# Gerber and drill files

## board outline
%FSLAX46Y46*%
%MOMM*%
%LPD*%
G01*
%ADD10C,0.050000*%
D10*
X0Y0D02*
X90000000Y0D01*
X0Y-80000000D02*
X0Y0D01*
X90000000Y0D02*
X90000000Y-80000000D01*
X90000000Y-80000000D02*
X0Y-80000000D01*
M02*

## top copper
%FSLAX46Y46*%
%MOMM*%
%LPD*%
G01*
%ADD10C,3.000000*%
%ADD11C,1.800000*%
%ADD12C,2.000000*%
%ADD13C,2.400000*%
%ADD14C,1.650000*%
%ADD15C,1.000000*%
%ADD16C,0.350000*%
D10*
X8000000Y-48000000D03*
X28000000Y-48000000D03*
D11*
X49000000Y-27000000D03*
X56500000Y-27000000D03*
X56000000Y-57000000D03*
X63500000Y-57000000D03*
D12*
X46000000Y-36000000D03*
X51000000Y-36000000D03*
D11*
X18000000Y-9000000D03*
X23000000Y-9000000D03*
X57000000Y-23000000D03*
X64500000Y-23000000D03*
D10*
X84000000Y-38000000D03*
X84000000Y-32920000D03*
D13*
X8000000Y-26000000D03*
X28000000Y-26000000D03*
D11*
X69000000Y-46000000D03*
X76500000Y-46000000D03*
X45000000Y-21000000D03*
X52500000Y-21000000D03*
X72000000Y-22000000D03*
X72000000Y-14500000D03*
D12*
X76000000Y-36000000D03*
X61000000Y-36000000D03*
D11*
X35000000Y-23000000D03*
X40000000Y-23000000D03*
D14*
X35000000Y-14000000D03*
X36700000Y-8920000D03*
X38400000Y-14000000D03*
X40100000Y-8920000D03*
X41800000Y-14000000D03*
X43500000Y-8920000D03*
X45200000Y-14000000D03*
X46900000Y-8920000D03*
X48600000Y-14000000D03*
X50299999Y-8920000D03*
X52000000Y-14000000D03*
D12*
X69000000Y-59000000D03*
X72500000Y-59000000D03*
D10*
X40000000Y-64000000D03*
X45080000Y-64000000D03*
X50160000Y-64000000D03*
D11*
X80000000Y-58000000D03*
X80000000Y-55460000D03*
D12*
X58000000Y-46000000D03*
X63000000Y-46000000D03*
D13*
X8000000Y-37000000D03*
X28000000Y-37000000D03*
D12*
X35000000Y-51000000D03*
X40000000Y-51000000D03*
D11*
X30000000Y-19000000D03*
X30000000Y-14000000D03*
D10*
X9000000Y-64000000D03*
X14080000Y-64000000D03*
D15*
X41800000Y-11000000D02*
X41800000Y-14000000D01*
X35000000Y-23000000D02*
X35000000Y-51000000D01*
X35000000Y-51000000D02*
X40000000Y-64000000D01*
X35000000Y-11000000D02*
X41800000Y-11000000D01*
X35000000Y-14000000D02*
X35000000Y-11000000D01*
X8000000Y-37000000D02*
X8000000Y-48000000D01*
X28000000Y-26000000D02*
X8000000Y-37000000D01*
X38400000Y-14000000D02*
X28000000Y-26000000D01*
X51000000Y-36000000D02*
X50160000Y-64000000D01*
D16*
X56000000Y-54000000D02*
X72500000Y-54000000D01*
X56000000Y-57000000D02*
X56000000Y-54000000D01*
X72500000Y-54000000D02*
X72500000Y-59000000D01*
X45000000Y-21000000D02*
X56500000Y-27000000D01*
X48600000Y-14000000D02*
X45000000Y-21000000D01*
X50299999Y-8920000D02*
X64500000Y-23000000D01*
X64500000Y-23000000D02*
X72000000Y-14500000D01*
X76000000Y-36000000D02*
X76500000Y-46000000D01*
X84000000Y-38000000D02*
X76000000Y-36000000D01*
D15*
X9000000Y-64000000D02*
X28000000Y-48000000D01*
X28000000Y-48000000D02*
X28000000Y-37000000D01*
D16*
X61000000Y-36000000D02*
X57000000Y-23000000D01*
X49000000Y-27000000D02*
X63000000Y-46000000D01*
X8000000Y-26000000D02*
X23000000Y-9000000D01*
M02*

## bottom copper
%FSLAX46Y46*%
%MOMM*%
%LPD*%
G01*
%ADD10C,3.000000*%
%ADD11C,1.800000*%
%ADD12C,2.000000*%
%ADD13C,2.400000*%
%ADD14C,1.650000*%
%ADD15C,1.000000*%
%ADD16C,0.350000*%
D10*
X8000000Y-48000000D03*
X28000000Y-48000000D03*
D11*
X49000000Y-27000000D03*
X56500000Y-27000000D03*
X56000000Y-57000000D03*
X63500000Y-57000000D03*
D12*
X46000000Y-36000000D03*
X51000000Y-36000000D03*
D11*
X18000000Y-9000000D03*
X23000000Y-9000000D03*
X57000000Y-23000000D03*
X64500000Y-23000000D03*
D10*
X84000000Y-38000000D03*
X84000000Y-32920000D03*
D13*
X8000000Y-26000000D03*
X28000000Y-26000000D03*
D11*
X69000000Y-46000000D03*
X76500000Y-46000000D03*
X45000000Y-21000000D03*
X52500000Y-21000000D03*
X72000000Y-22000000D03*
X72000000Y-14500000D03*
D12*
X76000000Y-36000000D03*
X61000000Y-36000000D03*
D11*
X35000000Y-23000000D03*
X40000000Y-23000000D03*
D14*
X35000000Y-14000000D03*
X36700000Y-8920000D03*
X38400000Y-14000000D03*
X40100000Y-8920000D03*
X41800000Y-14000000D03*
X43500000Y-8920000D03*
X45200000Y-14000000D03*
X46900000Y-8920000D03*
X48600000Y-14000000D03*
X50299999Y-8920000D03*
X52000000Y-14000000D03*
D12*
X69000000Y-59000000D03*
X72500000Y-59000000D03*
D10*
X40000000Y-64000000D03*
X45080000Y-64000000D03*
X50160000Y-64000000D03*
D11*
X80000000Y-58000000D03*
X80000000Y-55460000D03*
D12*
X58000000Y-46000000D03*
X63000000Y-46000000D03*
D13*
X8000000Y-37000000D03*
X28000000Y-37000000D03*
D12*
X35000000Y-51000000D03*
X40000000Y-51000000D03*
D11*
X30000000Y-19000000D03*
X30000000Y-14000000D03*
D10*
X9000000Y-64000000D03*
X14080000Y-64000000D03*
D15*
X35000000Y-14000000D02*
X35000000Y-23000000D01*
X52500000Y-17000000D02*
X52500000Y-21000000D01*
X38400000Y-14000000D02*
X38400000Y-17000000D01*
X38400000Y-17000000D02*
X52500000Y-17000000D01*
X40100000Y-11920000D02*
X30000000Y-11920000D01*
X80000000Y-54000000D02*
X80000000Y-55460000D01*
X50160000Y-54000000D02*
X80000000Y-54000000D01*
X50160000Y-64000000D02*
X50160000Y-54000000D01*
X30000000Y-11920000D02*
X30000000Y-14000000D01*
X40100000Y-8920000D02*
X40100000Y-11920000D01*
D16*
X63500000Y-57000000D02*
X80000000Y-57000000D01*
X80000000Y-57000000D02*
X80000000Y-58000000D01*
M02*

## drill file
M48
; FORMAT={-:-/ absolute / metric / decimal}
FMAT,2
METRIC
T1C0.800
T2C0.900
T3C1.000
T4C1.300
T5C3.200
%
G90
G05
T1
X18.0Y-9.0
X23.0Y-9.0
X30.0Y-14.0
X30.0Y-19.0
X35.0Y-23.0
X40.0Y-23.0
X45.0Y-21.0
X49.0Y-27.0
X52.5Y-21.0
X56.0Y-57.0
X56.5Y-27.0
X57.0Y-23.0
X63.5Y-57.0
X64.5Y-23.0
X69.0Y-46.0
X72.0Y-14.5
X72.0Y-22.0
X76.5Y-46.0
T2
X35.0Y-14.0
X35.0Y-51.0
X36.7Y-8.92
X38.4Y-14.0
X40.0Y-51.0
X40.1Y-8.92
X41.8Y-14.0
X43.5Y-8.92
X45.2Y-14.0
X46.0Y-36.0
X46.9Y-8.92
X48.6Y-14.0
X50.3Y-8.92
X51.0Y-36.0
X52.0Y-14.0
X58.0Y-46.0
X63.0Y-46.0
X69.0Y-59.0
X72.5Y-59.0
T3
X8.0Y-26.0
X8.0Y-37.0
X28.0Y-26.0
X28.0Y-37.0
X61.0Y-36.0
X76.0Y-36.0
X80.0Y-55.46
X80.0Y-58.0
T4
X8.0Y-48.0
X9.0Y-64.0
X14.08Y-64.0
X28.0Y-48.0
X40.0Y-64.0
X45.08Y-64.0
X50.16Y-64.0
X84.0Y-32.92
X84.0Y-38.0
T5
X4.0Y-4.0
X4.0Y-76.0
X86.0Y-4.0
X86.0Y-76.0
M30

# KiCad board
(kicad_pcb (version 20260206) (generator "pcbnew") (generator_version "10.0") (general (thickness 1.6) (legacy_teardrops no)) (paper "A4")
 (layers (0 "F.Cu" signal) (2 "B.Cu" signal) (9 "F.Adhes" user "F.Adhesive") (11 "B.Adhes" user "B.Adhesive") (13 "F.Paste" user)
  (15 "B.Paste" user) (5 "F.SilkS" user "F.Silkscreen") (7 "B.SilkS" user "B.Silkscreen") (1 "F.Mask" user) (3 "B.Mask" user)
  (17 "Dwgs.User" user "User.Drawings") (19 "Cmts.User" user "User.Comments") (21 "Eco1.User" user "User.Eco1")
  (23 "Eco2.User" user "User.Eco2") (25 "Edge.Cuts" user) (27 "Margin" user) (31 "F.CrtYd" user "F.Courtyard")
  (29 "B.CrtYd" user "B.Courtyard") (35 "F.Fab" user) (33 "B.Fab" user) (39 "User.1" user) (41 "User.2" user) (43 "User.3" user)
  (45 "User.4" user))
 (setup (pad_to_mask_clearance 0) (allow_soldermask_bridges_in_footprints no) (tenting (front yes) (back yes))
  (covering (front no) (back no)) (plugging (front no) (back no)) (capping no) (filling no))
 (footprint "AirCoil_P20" (layer "F.Cu") (at 8 48)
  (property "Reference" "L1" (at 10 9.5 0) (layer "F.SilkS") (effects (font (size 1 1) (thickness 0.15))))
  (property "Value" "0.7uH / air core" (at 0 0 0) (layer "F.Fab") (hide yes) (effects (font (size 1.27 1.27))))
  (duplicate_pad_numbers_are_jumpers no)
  (pad "1" thru_hole circle (at 0 0) (size 3 3) (drill 1.3) (layers "*.Cu" "*.Mask") (remove_unused_layers no) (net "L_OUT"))
  (pad "2" thru_hole circle (at 20 0) (size 3 3) (drill 1.3) (layers "*.Cu" "*.Mask") (remove_unused_layers no) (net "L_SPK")))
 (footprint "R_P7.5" (layer "F.Cu") (at 49 27)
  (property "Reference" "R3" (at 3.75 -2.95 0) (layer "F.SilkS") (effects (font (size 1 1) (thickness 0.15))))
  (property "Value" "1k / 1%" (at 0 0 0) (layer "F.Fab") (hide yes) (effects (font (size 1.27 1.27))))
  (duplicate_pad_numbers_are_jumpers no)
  (pad "1" thru_hole circle (at 0 0) (size 1.8 1.8) (drill 0.8) (layers "*.Cu" "*.Mask") (remove_unused_layers no) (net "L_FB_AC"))
  (pad "2" thru_hole circle (at 7.5 0) (size 1.8 1.8) (drill 0.8) (layers "*.Cu" "*.Mask") (remove_unused_layers no) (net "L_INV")))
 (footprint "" (layer "F.Cu") (at 4 4)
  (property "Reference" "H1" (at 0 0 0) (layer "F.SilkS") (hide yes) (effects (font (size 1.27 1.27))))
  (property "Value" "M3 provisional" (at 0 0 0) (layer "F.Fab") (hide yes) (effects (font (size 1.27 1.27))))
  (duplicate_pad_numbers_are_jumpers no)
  (pad "" np_thru_hole circle (at 0 0) (size 3.2 3.2) (drill 3.2) (layers "*.Cu" "*.Mask")))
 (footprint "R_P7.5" (layer "F.Cu") (at 56 57)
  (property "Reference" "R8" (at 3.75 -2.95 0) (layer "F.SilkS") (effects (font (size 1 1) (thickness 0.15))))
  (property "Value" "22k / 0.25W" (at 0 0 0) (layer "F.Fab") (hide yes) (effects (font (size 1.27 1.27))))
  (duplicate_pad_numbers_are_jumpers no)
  (pad "1" thru_hole circle (at 0 0) (size 1.8 1.8) (drill 0.8) (layers "*.Cu" "*.Mask") (remove_unused_layers no) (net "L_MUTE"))
  (pad "2" thru_hole circle (at 7.5 0) (size 1.8 1.8) (drill 0.8) (layers "*.Cu" "*.Mask") (remove_unused_layers no) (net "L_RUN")))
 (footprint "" (layer "F.Cu") (at 86 4)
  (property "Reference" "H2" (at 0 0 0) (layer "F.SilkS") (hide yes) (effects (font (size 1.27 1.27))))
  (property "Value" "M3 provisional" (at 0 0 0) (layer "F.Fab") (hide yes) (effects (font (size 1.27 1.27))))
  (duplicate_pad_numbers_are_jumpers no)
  (pad "" np_thru_hole circle (at 0 0) (size 3.2 3.2) (drill 3.2) (layers "*.Cu" "*.Mask")))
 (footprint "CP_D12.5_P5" (layer "F.Cu") (at 46 36)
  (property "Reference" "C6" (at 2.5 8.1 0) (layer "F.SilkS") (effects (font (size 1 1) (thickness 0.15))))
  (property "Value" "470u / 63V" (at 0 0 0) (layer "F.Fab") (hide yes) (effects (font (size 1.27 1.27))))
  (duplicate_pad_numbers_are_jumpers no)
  (pad "1" thru_hole circle (at 0 0) (size 2 2) (drill 0.9) (layers "*.Cu" "*.Mask") (remove_unused_layers no) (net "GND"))
  (pad "2" thru_hole circle (at 5 0) (size 2 2) (drill 0.9) (layers "*.Cu" "*.Mask") (remove_unused_layers no) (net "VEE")))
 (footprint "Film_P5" (layer "F.Cu") (at 18 9)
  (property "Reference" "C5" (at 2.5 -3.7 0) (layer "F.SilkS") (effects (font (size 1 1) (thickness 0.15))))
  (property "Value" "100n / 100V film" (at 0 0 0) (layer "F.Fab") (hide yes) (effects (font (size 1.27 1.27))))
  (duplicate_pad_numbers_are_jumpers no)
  (pad "1" thru_hole circle (at 0 0) (size 1.8 1.8) (drill 0.8) (layers "*.Cu" "*.Mask") (remove_unused_layers no) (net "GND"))
  (pad "2" thru_hole circle (at 5 0) (size 1.8 1.8) (drill 0.8) (layers "*.Cu" "*.Mask") (remove_unused_layers no) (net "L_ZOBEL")))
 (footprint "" (layer "F.Cu") (at 4 76)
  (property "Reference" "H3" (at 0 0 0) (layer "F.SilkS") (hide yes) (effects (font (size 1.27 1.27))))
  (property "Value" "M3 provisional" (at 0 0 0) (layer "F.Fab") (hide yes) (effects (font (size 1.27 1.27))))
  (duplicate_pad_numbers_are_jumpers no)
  (pad "" np_thru_hole circle (at 0 0) (size 3.2 3.2) (drill 3.2) (layers "*.Cu" "*.Mask")))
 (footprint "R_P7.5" (layer "F.Cu") (at 57 23)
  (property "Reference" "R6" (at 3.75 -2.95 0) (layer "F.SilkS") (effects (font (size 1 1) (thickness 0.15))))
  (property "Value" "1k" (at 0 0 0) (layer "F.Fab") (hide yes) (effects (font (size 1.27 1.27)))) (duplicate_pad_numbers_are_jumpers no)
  (pad "1" thru_hole circle (at 0 0) (size 1.8 1.8) (drill 0.8) (layers "*.Cu" "*.Mask") (remove_unused_layers no) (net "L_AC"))
  (pad "2" thru_hole circle (at 7.5 0) (size 1.8 1.8) (drill 0.8) (layers "*.Cu" "*.Mask") (remove_unused_layers no) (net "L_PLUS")))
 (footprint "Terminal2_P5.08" (layer "F.Cu") (at 84 38 90)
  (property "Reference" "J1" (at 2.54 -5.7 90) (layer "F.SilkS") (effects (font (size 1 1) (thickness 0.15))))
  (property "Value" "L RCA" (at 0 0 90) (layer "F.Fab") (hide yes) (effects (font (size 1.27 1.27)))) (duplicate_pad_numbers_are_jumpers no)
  (pad "1" thru_hole circle (at 0 0 90) (size 3 3) (drill 1.3) (layers "*.Cu" "*.Mask") (remove_unused_layers no) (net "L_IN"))
  (pad "2" thru_hole circle (at 5.08 0 90) (size 3 3) (drill 1.3) (layers "*.Cu" "*.Mask") (remove_unused_layers no) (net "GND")))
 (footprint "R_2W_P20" (layer "F.Cu") (at 8 26)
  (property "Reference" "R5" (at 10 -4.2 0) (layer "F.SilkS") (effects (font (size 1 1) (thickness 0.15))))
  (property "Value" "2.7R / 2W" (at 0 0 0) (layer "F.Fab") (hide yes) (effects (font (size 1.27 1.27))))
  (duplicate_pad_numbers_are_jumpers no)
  (pad "1" thru_hole circle (at 0 0) (size 2.4 2.4) (drill 1) (layers "*.Cu" "*.Mask") (remove_unused_layers no) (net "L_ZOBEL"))
  (pad "2" thru_hole circle (at 20 0) (size 2.4 2.4) (drill 1) (layers "*.Cu" "*.Mask") (remove_unused_layers no) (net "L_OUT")))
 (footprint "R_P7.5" (layer "F.Cu") (at 69 46)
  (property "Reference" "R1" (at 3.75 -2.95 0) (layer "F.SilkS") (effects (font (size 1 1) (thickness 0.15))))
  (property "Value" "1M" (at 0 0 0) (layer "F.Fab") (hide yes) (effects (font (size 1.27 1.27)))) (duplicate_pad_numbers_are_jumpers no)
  (pad "1" thru_hole circle (at 0 0) (size 1.8 1.8) (drill 0.8) (layers "*.Cu" "*.Mask") (remove_unused_layers no) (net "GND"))
  (pad "2" thru_hole circle (at 7.5 0) (size 1.8 1.8) (drill 0.8) (layers "*.Cu" "*.Mask") (remove_unused_layers no) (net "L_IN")))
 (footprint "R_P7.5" (layer "F.Cu") (at 45 21)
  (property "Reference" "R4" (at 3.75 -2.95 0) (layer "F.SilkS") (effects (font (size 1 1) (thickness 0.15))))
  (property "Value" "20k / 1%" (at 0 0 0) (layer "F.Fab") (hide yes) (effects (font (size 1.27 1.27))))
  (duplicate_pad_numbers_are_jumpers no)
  (pad "1" thru_hole circle (at 0 0) (size 1.8 1.8) (drill 0.8) (layers "*.Cu" "*.Mask") (remove_unused_layers no) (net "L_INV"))
  (pad "2" thru_hole circle (at 7.5 0) (size 1.8 1.8) (drill 0.8) (layers "*.Cu" "*.Mask") (remove_unused_layers no) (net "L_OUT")))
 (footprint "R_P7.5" (layer "F.Cu") (at 72 22 90)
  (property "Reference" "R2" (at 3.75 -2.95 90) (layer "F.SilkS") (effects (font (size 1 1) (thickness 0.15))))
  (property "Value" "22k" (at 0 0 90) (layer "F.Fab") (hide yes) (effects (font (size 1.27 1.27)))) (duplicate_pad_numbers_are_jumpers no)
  (pad "1" thru_hole circle (at 0 0 90) (size 1.8 1.8) (drill 0.8) (layers "*.Cu" "*.Mask") (remove_unused_layers no) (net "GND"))
  (pad "2" thru_hole circle (at 7.5 0 90) (size 1.8 1.8) (drill 0.8) (layers "*.Cu" "*.Mask") (remove_unused_layers no) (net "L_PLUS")))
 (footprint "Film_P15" (layer "F.Cu") (at 76 36 180)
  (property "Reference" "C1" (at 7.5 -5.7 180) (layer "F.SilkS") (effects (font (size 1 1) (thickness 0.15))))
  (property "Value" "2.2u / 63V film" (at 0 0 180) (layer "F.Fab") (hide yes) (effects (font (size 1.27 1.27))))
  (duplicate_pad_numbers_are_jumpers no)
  (pad "1" thru_hole circle (at 0 0 180) (size 2 2) (drill 1) (layers "*.Cu" "*.Mask") (remove_unused_layers no) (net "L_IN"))
  (pad "2" thru_hole circle (at 15 0 180) (size 2 2) (drill 1) (layers "*.Cu" "*.Mask") (remove_unused_layers no) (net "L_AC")))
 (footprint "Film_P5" (layer "F.Cu") (at 35 23)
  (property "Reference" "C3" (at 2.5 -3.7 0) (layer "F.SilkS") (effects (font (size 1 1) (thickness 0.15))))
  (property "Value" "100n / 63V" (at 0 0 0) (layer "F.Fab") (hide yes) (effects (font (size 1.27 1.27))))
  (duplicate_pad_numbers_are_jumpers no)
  (pad "1" thru_hole circle (at 0 0) (size 1.8 1.8) (drill 0.8) (layers "*.Cu" "*.Mask") (remove_unused_layers no) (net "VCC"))
  (pad "2" thru_hole circle (at 5 0) (size 1.8 1.8) (drill 0.8) (layers "*.Cu" "*.Mask") (remove_unused_layers no) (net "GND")))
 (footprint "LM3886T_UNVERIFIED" (layer "F.Cu") (at 35 14)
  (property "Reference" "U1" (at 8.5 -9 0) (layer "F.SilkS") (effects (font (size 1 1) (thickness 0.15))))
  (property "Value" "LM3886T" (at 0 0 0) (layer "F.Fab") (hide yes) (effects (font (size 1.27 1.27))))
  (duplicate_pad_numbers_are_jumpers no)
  (pad "1" thru_hole circle (at 0 0) (size 1.65 1.65) (drill 0.9) (layers "*.Cu" "*.Mask") (remove_unused_layers no) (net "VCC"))
  (pad "2" thru_hole circle (at 1.7 -5.08) (size 1.65 1.65) (drill 0.9) (layers "*.Cu" "*.Mask") (remove_unused_layers no)
   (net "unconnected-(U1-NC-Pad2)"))
  (pad "3" thru_hole circle (at 3.4 0) (size 1.65 1.65) (drill 0.9) (layers "*.Cu" "*.Mask") (remove_unused_layers no) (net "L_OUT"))
  (pad "4" thru_hole circle (at 5.1 -5.08) (size 1.65 1.65) (drill 0.9) (layers "*.Cu" "*.Mask") (remove_unused_layers no) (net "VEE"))
  (pad "5" thru_hole circle (at 6.8 0) (size 1.65 1.65) (drill 0.9) (layers "*.Cu" "*.Mask") (remove_unused_layers no) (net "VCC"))
  (pad "6" thru_hole circle (at 8.5 -5.08) (size 1.65 1.65) (drill 0.9) (layers "*.Cu" "*.Mask") (remove_unused_layers no)
   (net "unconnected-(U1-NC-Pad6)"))
  (pad "7" thru_hole circle (at 10.2 0) (size 1.65 1.65) (drill 0.9) (layers "*.Cu" "*.Mask") (remove_unused_layers no) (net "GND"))
  (pad "8" thru_hole circle (at 11.9 -5.08) (size 1.65 1.65) (drill 0.9) (layers "*.Cu" "*.Mask") (remove_unused_layers no) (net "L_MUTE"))
  (pad "9" thru_hole circle (at 13.6 0) (size 1.65 1.65) (drill 0.9) (layers "*.Cu" "*.Mask") (remove_unused_layers no) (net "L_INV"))
  (pad "10" thru_hole circle (at 15.299999 -5.08) (size 1.65 1.65) (drill 0.9) (layers "*.Cu" "*.Mask") (remove_unused_layers no)
   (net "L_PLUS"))
  (pad "11" thru_hole circle (at 17 0) (size 1.65 1.65) (drill 0.9) (layers "*.Cu" "*.Mask") (remove_unused_layers no)
   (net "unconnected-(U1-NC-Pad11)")))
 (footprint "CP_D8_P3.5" (layer "F.Cu") (at 69 59)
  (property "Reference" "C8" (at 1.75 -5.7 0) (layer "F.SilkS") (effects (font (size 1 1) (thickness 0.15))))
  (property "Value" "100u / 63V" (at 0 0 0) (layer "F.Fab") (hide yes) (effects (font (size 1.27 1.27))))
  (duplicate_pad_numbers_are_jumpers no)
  (pad "1" thru_hole circle (at 0 0) (size 2 2) (drill 0.9) (layers "*.Cu" "*.Mask") (remove_unused_layers no) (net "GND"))
  (pad "2" thru_hole circle (at 3.5 0) (size 2 2) (drill 0.9) (layers "*.Cu" "*.Mask") (remove_unused_layers no) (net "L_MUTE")))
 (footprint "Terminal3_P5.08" (layer "F.Cu") (at 40 64)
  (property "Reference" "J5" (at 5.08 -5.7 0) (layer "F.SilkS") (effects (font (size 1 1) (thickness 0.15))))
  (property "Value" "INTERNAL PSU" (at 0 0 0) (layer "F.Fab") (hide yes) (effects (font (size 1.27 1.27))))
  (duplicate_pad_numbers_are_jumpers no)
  (pad "1" thru_hole circle (at 0 0) (size 3 3) (drill 1.3) (layers "*.Cu" "*.Mask") (remove_unused_layers no) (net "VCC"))
  (pad "2" thru_hole circle (at 5.08 0) (size 3 3) (drill 1.3) (layers "*.Cu" "*.Mask") (remove_unused_layers no) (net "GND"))
  (pad "3" thru_hole circle (at 10.16 0) (size 3 3) (drill 1.3) (layers "*.Cu" "*.Mask") (remove_unused_layers no) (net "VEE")))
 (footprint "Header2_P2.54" (layer "F.Cu") (at 80 58 90)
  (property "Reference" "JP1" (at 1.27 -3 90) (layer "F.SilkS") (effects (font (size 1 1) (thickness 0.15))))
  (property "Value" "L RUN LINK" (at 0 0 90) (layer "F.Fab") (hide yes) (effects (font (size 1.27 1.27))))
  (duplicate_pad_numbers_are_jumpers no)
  (pad "1" thru_hole circle (at 0 0 90) (size 1.8 1.8) (drill 1) (layers "*.Cu" "*.Mask") (remove_unused_layers no) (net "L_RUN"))
  (pad "2" thru_hole circle (at 2.54 0 90) (size 1.8 1.8) (drill 1) (layers "*.Cu" "*.Mask") (remove_unused_layers no) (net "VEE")))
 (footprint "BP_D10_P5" (layer "F.Cu") (at 58 46)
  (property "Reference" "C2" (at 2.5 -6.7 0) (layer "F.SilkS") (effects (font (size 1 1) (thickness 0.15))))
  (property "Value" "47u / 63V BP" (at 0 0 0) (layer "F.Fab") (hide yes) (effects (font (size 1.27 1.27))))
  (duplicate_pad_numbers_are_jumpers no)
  (pad "1" thru_hole circle (at 0 0) (size 2 2) (drill 0.9) (layers "*.Cu" "*.Mask") (remove_unused_layers no) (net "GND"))
  (pad "2" thru_hole circle (at 5 0) (size 2 2) (drill 0.9) (layers "*.Cu" "*.Mask") (remove_unused_layers no) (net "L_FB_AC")))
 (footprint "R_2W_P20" (layer "F.Cu") (at 8 37)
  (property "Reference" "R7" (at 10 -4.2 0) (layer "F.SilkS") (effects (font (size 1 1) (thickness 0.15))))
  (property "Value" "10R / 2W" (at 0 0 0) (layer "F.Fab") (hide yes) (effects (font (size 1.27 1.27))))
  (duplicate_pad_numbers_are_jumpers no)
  (pad "1" thru_hole circle (at 0 0) (size 2.4 2.4) (drill 1) (layers "*.Cu" "*.Mask") (remove_unused_layers no) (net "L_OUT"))
  (pad "2" thru_hole circle (at 20 0) (size 2.4 2.4) (drill 1) (layers "*.Cu" "*.Mask") (remove_unused_layers no) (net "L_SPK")))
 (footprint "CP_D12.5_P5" (layer "F.Cu") (at 35 51)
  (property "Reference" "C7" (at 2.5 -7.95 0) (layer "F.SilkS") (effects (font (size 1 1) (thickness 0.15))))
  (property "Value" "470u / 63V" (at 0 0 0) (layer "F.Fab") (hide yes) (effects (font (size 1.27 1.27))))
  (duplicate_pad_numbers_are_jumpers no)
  (pad "1" thru_hole circle (at 0 0) (size 2 2) (drill 0.9) (layers "*.Cu" "*.Mask") (remove_unused_layers no) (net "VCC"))
  (pad "2" thru_hole circle (at 5 0) (size 2 2) (drill 0.9) (layers "*.Cu" "*.Mask") (remove_unused_layers no) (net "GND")))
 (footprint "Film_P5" (layer "F.Cu") (at 30 19 90)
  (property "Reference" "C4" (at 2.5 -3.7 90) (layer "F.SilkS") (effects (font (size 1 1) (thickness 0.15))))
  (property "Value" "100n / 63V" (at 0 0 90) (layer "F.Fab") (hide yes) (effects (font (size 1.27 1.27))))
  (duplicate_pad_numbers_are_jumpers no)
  (pad "1" thru_hole circle (at 0 0 90) (size 1.8 1.8) (drill 0.8) (layers "*.Cu" "*.Mask") (remove_unused_layers no) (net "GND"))
  (pad "2" thru_hole circle (at 5 0 90) (size 1.8 1.8) (drill 0.8) (layers "*.Cu" "*.Mask") (remove_unused_layers no) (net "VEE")))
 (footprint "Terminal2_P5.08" (layer "F.Cu") (at 9 64)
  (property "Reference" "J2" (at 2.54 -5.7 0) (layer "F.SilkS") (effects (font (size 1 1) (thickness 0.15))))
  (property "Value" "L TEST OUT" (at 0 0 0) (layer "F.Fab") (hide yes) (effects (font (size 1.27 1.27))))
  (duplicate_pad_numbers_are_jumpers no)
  (pad "1" thru_hole circle (at 0 0) (size 3 3) (drill 1.3) (layers "*.Cu" "*.Mask") (remove_unused_layers no) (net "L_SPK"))
  (pad "2" thru_hole circle (at 5.08 0) (size 3 3) (drill 1.3) (layers "*.Cu" "*.Mask") (remove_unused_layers no) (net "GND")))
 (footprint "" (layer "F.Cu") (at 86 76)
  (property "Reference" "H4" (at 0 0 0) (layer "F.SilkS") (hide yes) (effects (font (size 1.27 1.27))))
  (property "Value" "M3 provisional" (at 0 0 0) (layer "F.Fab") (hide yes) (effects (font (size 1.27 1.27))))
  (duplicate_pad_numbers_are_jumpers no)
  (pad "" np_thru_hole circle (at 0 0) (size 3.2 3.2) (drill 3.2) (layers "*.Cu" "*.Mask")))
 (gr_line (start 0 0) (end 90 0) (stroke (width 0.05) (type default)) (layer "Edge.Cuts"))
 (gr_line (start 0 80) (end 0 0) (stroke (width 0.05) (type default)) (layer "Edge.Cuts"))
 (gr_line (start 90 0) (end 90 80) (stroke (width 0.05) (type default)) (layer "Edge.Cuts"))
 (gr_line (start 90 80) (end 0 80) (stroke (width 0.05) (type default)) (layer "Edge.Cuts"))
 (segment (start 41.8 11) (end 41.8 14) (width 1) (layer "F.Cu") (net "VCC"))
 (segment (start 35 23) (end 35 51) (width 1) (layer "F.Cu") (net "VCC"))
 (segment (start 35 51) (end 40 64) (width 1) (layer "F.Cu") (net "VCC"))
 (segment (start 35 11) (end 41.8 11) (width 1) (layer "F.Cu") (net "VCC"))
 (segment (start 35 14) (end 35 11) (width 1) (layer "F.Cu") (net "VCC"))
 (segment (start 35 14) (end 35 23) (width 1) (layer "B.Cu") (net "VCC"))
 (segment (start 8 37) (end 8 48) (width 1) (layer "F.Cu") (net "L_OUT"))
 (segment (start 28 26) (end 8 37) (width 1) (layer "F.Cu") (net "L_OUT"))
 (segment (start 38.4 14) (end 28 26) (width 1) (layer "F.Cu") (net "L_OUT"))
 (segment (start 52.5 17) (end 52.5 21) (width 1) (layer "B.Cu") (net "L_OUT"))
 (segment (start 38.4 14) (end 38.4 17) (width 1) (layer "B.Cu") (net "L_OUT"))
 (segment (start 38.4 17) (end 52.5 17) (width 1) (layer "B.Cu") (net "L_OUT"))
 (segment (start 51 36) (end 50.16 64) (width 1) (layer "F.Cu") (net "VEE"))
 (segment (start 40.1 11.92) (end 30 11.92) (width 1) (layer "B.Cu") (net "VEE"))
 (segment (start 80 54) (end 80 55.46) (width 1) (layer "B.Cu") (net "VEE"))
 (segment (start 50.16 54) (end 80 54) (width 1) (layer "B.Cu") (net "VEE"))
 (segment (start 50.16 64) (end 50.16 54) (width 1) (layer "B.Cu") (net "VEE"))
 (segment (start 30 11.92) (end 30 14) (width 1) (layer "B.Cu") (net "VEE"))
 (segment (start 40.1 8.92) (end 40.1 11.92) (width 1) (layer "B.Cu") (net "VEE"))
 (segment (start 56 54) (end 72.5 54) (width 0.35) (layer "F.Cu") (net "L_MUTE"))
 (segment (start 56 57) (end 56 54) (width 0.35) (layer "F.Cu") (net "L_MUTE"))
 (segment (start 72.5 54) (end 72.5 59) (width 0.35) (layer "F.Cu") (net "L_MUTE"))
 (segment (start 45 21) (end 56.5 27) (width 0.35) (layer "F.Cu") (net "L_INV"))
 (segment (start 48.6 14) (end 45 21) (width 0.35) (layer "F.Cu") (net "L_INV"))
 (segment (start 50.299999 8.92) (end 64.5 23) (width 0.35) (layer "F.Cu") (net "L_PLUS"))
 (segment (start 64.5 23) (end 72 14.5) (width 0.35) (layer "F.Cu") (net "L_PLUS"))
 (segment (start 76 36) (end 76.5 46) (width 0.35) (layer "F.Cu") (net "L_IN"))
 (segment (start 84 38) (end 76 36) (width 0.35) (layer "F.Cu") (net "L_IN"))
 (segment (start 9 64) (end 28 48) (width 1) (layer "F.Cu") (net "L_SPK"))
 (segment (start 28 48) (end 28 37) (width 1) (layer "F.Cu") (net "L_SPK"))
 (segment (start 61 36) (end 57 23) (width 0.35) (layer "F.Cu") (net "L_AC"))
 (segment (start 49 27) (end 63 46) (width 0.35) (layer "F.Cu") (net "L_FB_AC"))
 (segment (start 8 26) (end 23 9) (width 0.35) (layer "F.Cu") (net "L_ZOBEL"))
 (segment (start 63.5 57) (end 80 57) (width 0.35) (layer "B.Cu") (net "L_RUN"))
 (segment (start 80 57) (end 80 58) (width 0.35) (layer "B.Cu") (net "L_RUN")))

